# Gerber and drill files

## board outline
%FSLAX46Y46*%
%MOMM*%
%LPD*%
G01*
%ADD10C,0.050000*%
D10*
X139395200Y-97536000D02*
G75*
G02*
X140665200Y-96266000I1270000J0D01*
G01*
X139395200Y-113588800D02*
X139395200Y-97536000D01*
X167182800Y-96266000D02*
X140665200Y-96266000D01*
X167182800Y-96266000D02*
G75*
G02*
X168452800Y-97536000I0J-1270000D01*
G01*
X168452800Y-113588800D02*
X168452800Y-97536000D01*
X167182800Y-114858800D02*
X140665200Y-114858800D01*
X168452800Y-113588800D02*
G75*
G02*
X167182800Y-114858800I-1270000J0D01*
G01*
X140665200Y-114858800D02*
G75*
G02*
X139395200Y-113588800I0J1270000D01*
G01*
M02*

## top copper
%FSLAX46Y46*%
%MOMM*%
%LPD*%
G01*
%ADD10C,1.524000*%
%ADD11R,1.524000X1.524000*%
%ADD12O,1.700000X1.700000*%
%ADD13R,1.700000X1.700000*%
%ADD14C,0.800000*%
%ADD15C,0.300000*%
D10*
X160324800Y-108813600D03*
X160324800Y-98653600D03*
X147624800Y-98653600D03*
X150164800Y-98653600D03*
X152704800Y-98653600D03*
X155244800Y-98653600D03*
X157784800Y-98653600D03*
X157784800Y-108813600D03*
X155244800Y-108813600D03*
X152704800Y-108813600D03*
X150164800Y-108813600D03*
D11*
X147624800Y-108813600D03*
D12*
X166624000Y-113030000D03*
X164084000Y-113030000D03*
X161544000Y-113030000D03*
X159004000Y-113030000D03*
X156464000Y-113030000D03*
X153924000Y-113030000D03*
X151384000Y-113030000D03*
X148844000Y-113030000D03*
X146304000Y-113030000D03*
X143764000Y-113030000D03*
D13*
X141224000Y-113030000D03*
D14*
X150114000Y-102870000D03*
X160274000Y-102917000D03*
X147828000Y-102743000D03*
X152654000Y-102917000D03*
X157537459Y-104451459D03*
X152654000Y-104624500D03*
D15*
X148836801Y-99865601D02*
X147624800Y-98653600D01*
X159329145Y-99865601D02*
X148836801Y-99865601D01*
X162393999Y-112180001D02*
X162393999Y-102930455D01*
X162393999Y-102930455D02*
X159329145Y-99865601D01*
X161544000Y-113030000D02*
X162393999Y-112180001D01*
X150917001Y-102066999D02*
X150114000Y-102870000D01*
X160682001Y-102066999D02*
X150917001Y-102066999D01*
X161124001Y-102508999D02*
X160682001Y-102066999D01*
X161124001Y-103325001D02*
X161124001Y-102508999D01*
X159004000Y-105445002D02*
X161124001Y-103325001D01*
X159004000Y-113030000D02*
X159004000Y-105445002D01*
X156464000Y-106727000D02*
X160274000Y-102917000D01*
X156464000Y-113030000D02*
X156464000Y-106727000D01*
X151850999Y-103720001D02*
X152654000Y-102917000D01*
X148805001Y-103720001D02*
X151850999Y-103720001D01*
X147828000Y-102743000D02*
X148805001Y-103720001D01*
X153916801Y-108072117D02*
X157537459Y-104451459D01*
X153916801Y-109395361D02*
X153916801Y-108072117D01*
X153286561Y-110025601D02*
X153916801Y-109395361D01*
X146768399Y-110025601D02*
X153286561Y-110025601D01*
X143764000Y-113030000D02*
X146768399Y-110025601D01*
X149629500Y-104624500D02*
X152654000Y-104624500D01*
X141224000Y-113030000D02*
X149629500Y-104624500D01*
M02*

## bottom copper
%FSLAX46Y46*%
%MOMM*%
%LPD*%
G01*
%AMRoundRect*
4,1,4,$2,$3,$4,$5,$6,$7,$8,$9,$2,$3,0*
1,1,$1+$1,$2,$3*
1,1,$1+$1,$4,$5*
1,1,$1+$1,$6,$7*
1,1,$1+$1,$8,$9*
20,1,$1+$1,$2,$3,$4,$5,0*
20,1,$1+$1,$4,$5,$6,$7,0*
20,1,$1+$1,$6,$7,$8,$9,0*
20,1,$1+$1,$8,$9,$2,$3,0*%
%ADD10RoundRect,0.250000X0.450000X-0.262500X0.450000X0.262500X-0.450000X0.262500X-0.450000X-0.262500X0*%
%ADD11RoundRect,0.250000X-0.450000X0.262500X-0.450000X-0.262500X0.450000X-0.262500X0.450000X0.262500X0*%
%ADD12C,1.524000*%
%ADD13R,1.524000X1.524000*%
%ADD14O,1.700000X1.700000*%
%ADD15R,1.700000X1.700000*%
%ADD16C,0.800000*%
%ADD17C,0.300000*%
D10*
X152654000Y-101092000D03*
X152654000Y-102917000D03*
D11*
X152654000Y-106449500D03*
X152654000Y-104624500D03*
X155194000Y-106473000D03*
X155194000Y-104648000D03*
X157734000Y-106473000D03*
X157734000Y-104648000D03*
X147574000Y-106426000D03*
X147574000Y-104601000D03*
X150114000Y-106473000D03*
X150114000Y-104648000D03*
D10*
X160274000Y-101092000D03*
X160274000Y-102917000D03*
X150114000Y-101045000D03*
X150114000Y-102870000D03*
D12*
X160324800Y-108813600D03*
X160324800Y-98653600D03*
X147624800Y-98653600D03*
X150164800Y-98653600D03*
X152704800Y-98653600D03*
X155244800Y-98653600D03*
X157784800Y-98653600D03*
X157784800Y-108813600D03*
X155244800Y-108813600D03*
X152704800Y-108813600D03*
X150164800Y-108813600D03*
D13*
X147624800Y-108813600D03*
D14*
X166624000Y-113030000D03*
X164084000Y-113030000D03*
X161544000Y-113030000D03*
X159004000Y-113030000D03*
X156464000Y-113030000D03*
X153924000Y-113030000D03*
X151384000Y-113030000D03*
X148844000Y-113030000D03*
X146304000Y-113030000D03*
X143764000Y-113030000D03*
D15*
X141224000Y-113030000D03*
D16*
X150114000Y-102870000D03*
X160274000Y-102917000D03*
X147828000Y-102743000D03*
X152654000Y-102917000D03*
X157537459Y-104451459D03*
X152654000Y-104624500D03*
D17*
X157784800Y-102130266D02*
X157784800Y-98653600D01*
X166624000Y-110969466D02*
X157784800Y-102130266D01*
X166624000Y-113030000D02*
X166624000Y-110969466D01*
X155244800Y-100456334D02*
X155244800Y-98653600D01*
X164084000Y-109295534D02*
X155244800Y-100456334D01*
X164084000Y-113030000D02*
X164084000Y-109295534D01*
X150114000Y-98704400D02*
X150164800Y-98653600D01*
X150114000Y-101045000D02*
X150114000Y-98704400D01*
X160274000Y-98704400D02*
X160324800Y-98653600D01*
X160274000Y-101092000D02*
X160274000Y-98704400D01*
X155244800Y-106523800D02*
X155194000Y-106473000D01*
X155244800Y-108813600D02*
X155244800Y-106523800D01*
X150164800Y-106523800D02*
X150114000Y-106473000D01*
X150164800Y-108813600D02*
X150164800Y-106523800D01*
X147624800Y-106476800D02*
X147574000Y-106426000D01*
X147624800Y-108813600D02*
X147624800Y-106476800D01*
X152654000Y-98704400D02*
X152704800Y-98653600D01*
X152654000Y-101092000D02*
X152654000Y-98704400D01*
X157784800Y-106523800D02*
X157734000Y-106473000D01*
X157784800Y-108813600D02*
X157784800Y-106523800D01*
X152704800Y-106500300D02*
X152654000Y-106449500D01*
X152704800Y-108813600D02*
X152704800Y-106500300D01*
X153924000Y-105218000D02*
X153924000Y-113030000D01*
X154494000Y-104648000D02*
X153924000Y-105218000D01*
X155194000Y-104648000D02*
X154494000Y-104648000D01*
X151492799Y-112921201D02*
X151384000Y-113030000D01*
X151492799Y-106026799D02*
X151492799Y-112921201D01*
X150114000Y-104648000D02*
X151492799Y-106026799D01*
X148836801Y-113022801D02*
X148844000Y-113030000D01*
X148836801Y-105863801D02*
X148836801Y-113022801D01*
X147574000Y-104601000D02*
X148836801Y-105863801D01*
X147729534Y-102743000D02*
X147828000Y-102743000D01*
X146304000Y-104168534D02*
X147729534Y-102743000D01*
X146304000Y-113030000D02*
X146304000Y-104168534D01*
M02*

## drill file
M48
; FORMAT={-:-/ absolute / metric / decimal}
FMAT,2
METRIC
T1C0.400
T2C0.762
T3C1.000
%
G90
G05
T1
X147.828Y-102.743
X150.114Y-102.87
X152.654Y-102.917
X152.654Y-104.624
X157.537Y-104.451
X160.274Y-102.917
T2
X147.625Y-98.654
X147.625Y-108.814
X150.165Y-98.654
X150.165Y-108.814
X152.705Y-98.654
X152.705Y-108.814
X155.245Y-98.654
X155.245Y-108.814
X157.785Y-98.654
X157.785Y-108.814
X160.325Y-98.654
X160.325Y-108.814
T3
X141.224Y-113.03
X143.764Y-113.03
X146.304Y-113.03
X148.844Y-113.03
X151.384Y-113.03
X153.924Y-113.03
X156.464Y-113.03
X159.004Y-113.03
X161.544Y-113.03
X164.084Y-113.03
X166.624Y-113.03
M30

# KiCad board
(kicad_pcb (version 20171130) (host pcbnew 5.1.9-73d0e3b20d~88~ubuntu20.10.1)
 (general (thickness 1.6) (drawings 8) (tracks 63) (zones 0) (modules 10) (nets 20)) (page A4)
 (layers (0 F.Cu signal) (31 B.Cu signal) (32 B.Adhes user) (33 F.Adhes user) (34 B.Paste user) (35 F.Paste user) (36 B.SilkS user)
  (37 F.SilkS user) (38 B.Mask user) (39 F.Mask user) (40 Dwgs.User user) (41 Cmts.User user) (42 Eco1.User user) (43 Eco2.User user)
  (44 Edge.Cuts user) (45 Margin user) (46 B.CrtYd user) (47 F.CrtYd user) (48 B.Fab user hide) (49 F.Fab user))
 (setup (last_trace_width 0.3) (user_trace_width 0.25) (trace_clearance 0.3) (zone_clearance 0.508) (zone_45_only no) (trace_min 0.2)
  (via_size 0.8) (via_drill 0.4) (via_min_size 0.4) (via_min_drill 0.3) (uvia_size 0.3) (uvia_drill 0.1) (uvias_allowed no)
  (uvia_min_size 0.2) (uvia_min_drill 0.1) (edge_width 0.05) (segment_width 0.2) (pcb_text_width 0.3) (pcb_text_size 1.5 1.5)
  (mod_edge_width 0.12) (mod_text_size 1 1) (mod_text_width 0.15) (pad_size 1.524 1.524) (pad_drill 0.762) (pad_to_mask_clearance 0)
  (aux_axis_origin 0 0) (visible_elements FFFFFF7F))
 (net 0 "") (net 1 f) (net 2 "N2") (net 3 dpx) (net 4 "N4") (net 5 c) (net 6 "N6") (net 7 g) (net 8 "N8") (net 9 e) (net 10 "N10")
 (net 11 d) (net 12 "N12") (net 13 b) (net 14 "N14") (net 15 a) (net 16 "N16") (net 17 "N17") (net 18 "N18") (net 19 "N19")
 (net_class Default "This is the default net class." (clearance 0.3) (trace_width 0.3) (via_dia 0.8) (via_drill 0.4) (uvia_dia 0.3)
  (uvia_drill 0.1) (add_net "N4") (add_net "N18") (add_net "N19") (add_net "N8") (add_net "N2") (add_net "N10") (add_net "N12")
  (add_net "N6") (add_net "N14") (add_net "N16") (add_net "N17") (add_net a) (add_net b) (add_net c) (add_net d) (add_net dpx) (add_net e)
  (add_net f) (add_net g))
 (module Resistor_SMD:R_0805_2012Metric (layer B.Cu) (at 152.654 102.0045 90)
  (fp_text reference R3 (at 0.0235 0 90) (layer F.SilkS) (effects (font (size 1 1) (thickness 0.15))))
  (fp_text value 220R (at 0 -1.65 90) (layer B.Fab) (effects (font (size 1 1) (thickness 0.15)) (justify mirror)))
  (pad 2 smd roundrect (at 0.9125 0 90) (size 1.025 1.4) (layers B.Cu B.Paste B.Mask) (roundrect_rratio 0.243902) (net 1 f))
  (pad 1 smd roundrect (at -0.9125 0 90) (size 1.025 1.4) (layers B.Cu B.Paste B.Mask) (roundrect_rratio 0.243902) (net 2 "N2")))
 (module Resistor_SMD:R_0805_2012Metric (layer B.Cu) (at 152.654 105.537 270)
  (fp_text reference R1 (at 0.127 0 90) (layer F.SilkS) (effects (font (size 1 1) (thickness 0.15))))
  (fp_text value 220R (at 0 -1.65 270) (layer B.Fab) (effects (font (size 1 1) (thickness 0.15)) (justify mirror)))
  (pad 2 smd roundrect (at 0.9125 0 270) (size 1.025 1.4) (layers B.Cu B.Paste B.Mask) (roundrect_rratio 0.243902) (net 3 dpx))
  (pad 1 smd roundrect (at -0.9125 0 270) (size 1.025 1.4) (layers B.Cu B.Paste B.Mask) (roundrect_rratio 0.243902) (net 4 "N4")))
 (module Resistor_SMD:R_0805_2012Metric (layer B.Cu) (at 155.194 105.5605 270)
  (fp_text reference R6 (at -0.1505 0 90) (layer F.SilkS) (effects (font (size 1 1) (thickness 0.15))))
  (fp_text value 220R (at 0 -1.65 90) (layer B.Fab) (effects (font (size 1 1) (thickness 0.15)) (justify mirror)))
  (pad 2 smd roundrect (at 0.9125 0 270) (size 1.025 1.4) (layers B.Cu B.Paste B.Mask) (roundrect_rratio 0.243902) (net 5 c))
  (pad 1 smd roundrect (at -0.9125 0 270) (size 1.025 1.4) (layers B.Cu B.Paste B.Mask) (roundrect_rratio 0.243902) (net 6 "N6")))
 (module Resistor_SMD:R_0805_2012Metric (layer B.Cu) (at 157.734 105.5605 270)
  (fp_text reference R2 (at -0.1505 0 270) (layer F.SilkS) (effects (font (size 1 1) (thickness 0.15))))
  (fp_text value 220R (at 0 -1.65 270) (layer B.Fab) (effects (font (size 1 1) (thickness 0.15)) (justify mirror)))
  (pad 2 smd roundrect (at 0.9125 0 270) (size 1.025 1.4) (layers B.Cu B.Paste B.Mask) (roundrect_rratio 0.243902) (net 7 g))
  (pad 1 smd roundrect (at -0.9125 0 270) (size 1.025 1.4) (layers B.Cu B.Paste B.Mask) (roundrect_rratio 0.243902) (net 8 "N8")))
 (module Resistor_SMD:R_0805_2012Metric (layer B.Cu) (at 147.574 105.5135 270)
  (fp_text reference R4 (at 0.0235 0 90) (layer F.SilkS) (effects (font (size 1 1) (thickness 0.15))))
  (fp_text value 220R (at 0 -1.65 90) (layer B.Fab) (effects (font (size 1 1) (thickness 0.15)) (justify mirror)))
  (pad 2 smd roundrect (at 0.9125 0 270) (size 1.025 1.4) (layers B.Cu B.Paste B.Mask) (roundrect_rratio 0.243902) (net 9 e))
  (pad 1 smd roundrect (at -0.9125 0 270) (size 1.025 1.4) (layers B.Cu B.Paste B.Mask) (roundrect_rratio 0.243902) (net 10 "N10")))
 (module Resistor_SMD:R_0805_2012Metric (layer B.Cu) (at 150.114 105.5605 270)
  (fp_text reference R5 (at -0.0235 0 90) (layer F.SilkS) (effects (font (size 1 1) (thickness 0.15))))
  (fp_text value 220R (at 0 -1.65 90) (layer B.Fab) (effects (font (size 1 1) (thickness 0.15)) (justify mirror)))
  (pad 2 smd roundrect (at 0.9125 0 270) (size 1.025 1.4) (layers B.Cu B.Paste B.Mask) (roundrect_rratio 0.243902) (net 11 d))
  (pad 1 smd roundrect (at -0.9125 0 270) (size 1.025 1.4) (layers B.Cu B.Paste B.Mask) (roundrect_rratio 0.243902) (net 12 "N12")))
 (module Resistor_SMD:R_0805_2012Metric (layer B.Cu) (at 160.274 102.0045 90)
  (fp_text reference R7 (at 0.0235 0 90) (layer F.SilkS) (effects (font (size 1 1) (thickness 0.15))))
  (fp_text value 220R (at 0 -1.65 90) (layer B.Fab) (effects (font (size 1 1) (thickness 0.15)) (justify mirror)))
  (pad 2 smd roundrect (at 0.9125 0 90) (size 1.025 1.4) (layers B.Cu B.Paste B.Mask) (roundrect_rratio 0.243902) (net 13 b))
  (pad 1 smd roundrect (at -0.9125 0 90) (size 1.025 1.4) (layers B.Cu B.Paste B.Mask) (roundrect_rratio 0.243902) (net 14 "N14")))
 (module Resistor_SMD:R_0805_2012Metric (layer B.Cu) (at 150.114 101.9575 90)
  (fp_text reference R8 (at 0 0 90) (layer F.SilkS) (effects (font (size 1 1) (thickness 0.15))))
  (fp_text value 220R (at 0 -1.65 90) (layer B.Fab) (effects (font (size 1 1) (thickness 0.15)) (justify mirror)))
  (pad 2 smd roundrect (at 0.9125 0 90) (size 1.025 1.4) (layers B.Cu B.Paste B.Mask) (roundrect_rratio 0.243902) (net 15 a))
  (pad 1 smd roundrect (at -0.9125 0 90) (size 1.025 1.4) (layers B.Cu B.Paste B.Mask) (roundrect_rratio 0.243902) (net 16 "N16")))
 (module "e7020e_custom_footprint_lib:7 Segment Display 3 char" (layer F.Cu) (at 147.6248 98.6536)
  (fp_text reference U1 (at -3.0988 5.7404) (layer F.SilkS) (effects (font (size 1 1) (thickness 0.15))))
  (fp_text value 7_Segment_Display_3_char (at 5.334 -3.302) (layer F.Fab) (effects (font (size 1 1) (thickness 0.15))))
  (pad 6 thru_hole circle (at 12.7 10.16) (size 1.524 1.524) (drill 0.762) (layers *.Cu *.Mask))
  (pad 7 thru_hole circle (at 12.7 0) (size 1.524 1.524) (drill 0.762) (layers *.Cu *.Mask) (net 13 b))
  (pad 12 thru_hole circle (at 0 0) (size 1.524 1.524) (drill 0.762) (layers *.Cu *.Mask) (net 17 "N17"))
  (pad 11 thru_hole circle (at 2.54 0) (size 1.524 1.524) (drill 0.762) (layers *.Cu *.Mask) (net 15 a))
  (pad 10 thru_hole circle (at 5.08 0) (size 1.524 1.524) (drill 0.762) (layers *.Cu *.Mask) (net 1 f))
  (pad 9 thru_hole circle (at 7.62 0) (size 1.524 1.524) (drill 0.762) (layers *.Cu *.Mask) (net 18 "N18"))
  (pad 8 thru_hole circle (at 10.16 0) (size 1.524 1.524) (drill 0.762) (layers *.Cu *.Mask) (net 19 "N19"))
  (pad 5 thru_hole circle (at 10.16 10.16) (size 1.524 1.524) (drill 0.762) (layers *.Cu *.Mask) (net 7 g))
  (pad 4 thru_hole circle (at 7.62 10.16) (size 1.524 1.524) (drill 0.762) (layers *.Cu *.Mask) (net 5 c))
  (pad 3 thru_hole circle (at 5.08 10.16) (size 1.524 1.524) (drill 0.762) (layers *.Cu *.Mask) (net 3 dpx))
  (pad 2 thru_hole circle (at 2.54 10.16) (size 1.524 1.524) (drill 0.762) (layers *.Cu *.Mask) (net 11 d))
  (pad 1 thru_hole rect (at 0 10.16) (size 1.524 1.524) (drill 0.762) (layers *.Cu *.Mask) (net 9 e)))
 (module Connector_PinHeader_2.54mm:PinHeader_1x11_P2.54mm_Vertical (layer B.Cu) (at 141.224 113.03 270)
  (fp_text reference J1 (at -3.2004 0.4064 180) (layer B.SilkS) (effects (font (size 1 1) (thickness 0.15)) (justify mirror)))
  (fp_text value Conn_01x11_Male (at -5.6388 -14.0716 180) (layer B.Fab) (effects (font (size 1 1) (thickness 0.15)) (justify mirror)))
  (pad 11 thru_hole oval (at 0 -25.4 270) (size 1.7 1.7) (drill 1) (layers *.Cu *.Mask) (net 19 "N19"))
  (pad 10 thru_hole oval (at 0 -22.86 270) (size 1.7 1.7) (drill 1) (layers *.Cu *.Mask) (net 18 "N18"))
  (pad 9 thru_hole oval (at 0 -20.32 270) (size 1.7 1.7) (drill 1) (layers *.Cu *.Mask) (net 17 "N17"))
  (pad 8 thru_hole oval (at 0 -17.78 270) (size 1.7 1.7) (drill 1) (layers *.Cu *.Mask) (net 16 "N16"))
  (pad 7 thru_hole oval (at 0 -15.24 270) (size 1.7 1.7) (drill 1) (layers *.Cu *.Mask) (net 14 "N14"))
  (pad 6 thru_hole oval (at 0 -12.7 270) (size 1.7 1.7) (drill 1) (layers *.Cu *.Mask) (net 6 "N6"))
  (pad 5 thru_hole oval (at 0 -10.16 270) (size 1.7 1.7) (drill 1) (layers *.Cu *.Mask) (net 12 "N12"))
  (pad 4 thru_hole oval (at 0 -7.62 270) (size 1.7 1.7) (drill 1) (layers *.Cu *.Mask) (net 10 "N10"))
  (pad 3 thru_hole oval (at 0 -5.08 270) (size 1.7 1.7) (drill 1) (layers *.Cu *.Mask) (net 2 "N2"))
  (pad 2 thru_hole oval (at 0 -2.54 270) (size 1.7 1.7) (drill 1) (layers *.Cu *.Mask) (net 8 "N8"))
  (pad 1 thru_hole rect (at 0 0 270) (size 1.7 1.7) (drill 1) (layers *.Cu *.Mask) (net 4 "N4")))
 (gr_arc (start 140.6652 97.536) (end 140.6652 96.266) (angle -90) (layer Edge.Cuts) (width 0.05))
 (gr_line (start 139.3952 113.5888) (end 139.3952 97.536) (layer Edge.Cuts) (width 0.05))
 (gr_line (start 167.1828 96.266) (end 140.6652 96.266) (layer Edge.Cuts) (width 0.05))
 (gr_arc (start 167.1828 97.536) (end 168.4528 97.536) (angle -90) (layer Edge.Cuts) (width 0.05))
 (gr_line (start 168.4528 113.5888) (end 168.4528 97.536) (layer Edge.Cuts) (width 0.05))
 (gr_line (start 167.1828 114.8588) (end 140.6652 114.8588) (layer Edge.Cuts) (width 0.05))
 (gr_arc (start 167.1828 113.5888) (end 167.1828 114.8588) (angle -90) (layer Edge.Cuts) (width 0.05))
 (gr_arc (start 140.6652 113.5888) (end 139.3952 113.5888) (angle -90) (layer Edge.Cuts) (width 0.05))
 (segment (start 157.7848 102.130266) (end 157.7848 98.6536) (width 0.3) (layer B.Cu) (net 19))
 (segment (start 166.624 110.969466) (end 157.7848 102.130266) (width 0.3) (layer B.Cu) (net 19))
 (segment (start 166.624 113.03) (end 166.624 110.969466) (width 0.3) (layer B.Cu) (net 19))
 (segment (start 155.2448 100.456334) (end 155.2448 98.6536) (width 0.3) (layer B.Cu) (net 18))
 (segment (start 164.084 109.295534) (end 155.2448 100.456334) (width 0.3) (layer B.Cu) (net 18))
 (segment (start 164.084 113.03) (end 164.084 109.295534) (width 0.3) (layer B.Cu) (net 18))
 (segment (start 148.836801 99.865601) (end 147.6248 98.6536) (width 0.3) (layer F.Cu) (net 17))
 (segment (start 159.329145 99.865601) (end 148.836801 99.865601) (width 0.3) (layer F.Cu) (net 17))
 (segment (start 162.393999 112.180001) (end 162.393999 102.930455) (width 0.3) (layer F.Cu) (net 17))
 (segment (start 162.393999 102.930455) (end 159.329145 99.865601) (width 0.3) (layer F.Cu) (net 17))
 (segment (start 161.544 113.03) (end 162.393999 112.180001) (width 0.3) (layer F.Cu) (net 17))
 (segment (start 150.114 98.7044) (end 150.1648 98.6536) (width 0.3) (layer B.Cu) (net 15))
 (segment (start 150.114 101.045) (end 150.114 98.7044) (width 0.3) (layer B.Cu) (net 15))
 (segment (start 160.274 98.7044) (end 160.3248 98.6536) (width 0.3) (layer B.Cu) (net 13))
 (segment (start 160.274 101.092) (end 160.274 98.7044) (width 0.3) (layer B.Cu) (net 13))
 (segment (start 155.2448 106.5238) (end 155.194 106.473) (width 0.3) (layer B.Cu) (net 5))
 (segment (start 155.2448 108.8136) (end 155.2448 106.5238) (width 0.3) (layer B.Cu) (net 5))
 (segment (start 150.1648 106.5238) (end 150.114 106.473) (width 0.3) (layer B.Cu) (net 11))
 (segment (start 150.1648 108.8136) (end 150.1648 106.5238) (width 0.3) (layer B.Cu) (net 11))
 (segment (start 147.6248 106.4768) (end 147.574 106.426) (width 0.3) (layer B.Cu) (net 9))
 (segment (start 147.6248 108.8136) (end 147.6248 106.4768) (width 0.3) (layer B.Cu) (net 9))
 (segment (start 152.654 98.7044) (end 152.7048 98.6536) (width 0.3) (layer B.Cu) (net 1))
 (segment (start 152.654 101.092) (end 152.654 98.7044) (width 0.3) (layer B.Cu) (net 1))
 (segment (start 157.7848 106.5238) (end 157.734 106.473) (width 0.3) (layer B.Cu) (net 7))
 (segment (start 157.7848 108.8136) (end 157.7848 106.5238) (width 0.3) (layer B.Cu) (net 7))
 (segment (start 152.7048 106.5003) (end 152.654 106.4495) (width 0.3) (layer B.Cu) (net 3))
 (segment (start 152.7048 108.8136) (end 152.7048 106.5003) (width 0.3) (layer B.Cu) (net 3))
 (segment (start 150.917001 102.066999) (end 150.114 102.87) (width 0.3) (layer F.Cu) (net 16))
 (segment (start 160.682001 102.066999) (end 150.917001 102.066999) (width 0.3) (layer F.Cu) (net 16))
 (segment (start 161.124001 102.508999) (end 160.682001 102.066999) (width 0.3) (layer F.Cu) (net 16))
 (segment (start 161.124001 103.325001) (end 161.124001 102.508999) (width 0.3) (layer F.Cu) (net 16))
 (segment (start 159.004 105.445002) (end 161.124001 103.325001) (width 0.3) (layer F.Cu) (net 16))
 (via (at 150.114 102.87) (size 0.8) (drill 0.4) (layers F.Cu B.Cu) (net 16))
 (segment (start 159.004 113.03) (end 159.004 105.445002) (width 0.3) (layer F.Cu) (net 16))
 (via (at 160.274 102.917) (size 0.8) (drill 0.4) (layers F.Cu B.Cu) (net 14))
 (segment (start 156.464 106.727) (end 160.274 102.917) (width 0.3) (layer F.Cu) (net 14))
 (segment (start 156.464 113.03) (end 156.464 106.727) (width 0.3) (layer F.Cu) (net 14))
 (segment (start 153.924 105.218) (end 153.924 113.03) (width 0.3) (layer B.Cu) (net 6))
 (segment (start 154.494 104.648) (end 153.924 105.218) (width 0.3) (layer B.Cu) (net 6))
 (segment (start 155.194 104.648) (end 154.494 104.648) (width 0.3) (layer B.Cu) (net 6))
 (segment (start 151.492799 112.921201) (end 151.384 113.03) (width 0.3) (layer B.Cu) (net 12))
 (segment (start 151.492799 106.026799) (end 151.492799 112.921201) (width 0.3) (layer B.Cu) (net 12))
 (segment (start 150.114 104.648) (end 151.492799 106.026799) (width 0.3) (layer B.Cu) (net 12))
 (segment (start 148.836801 113.022801) (end 148.844 113.03) (width 0.3) (layer B.Cu) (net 10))
 (segment (start 148.836801 105.863801) (end 148.836801 113.022801) (width 0.3) (layer B.Cu) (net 10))
 (segment (start 147.574 104.601) (end 148.836801 105.863801) (width 0.3) (layer B.Cu) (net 10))
 (via (at 147.828 102.743) (size 0.8) (drill 0.4) (layers F.Cu B.Cu) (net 2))
 (segment (start 147.729534 102.743) (end 147.828 102.743) (width 0.3) (layer B.Cu) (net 2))
 (segment (start 146.304 104.168534) (end 147.729534 102.743) (width 0.3) (layer B.Cu) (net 2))
 (segment (start 146.304 113.03) (end 146.304 104.168534) (width 0.3) (layer B.Cu) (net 2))
 (via (at 152.654 102.917) (size 0.8) (drill 0.4) (layers F.Cu B.Cu) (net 2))
 (segment (start 151.850999 103.720001) (end 152.654 102.917) (width 0.3) (layer F.Cu) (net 2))
 (segment (start 148.805001 103.720001) (end 151.850999 103.720001) (width 0.3) (layer F.Cu) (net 2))
 (segment (start 147.828 102.743) (end 148.805001 103.720001) (width 0.3) (layer F.Cu) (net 2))
 (via (at 157.537459 104.451459) (size 0.8) (drill 0.4) (layers F.Cu B.Cu) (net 8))
 (segment (start 153.916801 108.072117) (end 157.537459 104.451459) (width 0.3) (layer F.Cu) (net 8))
 (segment (start 153.916801 109.395361) (end 153.916801 108.072117) (width 0.3) (layer F.Cu) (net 8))
 (segment (start 153.286561 110.025601) (end 153.916801 109.395361) (width 0.3) (layer F.Cu) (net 8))
 (segment (start 146.768399 110.025601) (end 153.286561 110.025601) (width 0.3) (layer F.Cu) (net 8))
 (segment (start 143.764 113.03) (end 146.768399 110.025601) (width 0.3) (layer F.Cu) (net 8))
 (via (at 152.654 104.6245) (size 0.8) (drill 0.4) (layers F.Cu B.Cu) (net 4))
 (segment (start 149.6295 104.6245) (end 152.654 104.6245) (width 0.3) (layer F.Cu) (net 4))
 (segment (start 141.224 113.03) (end 149.6295 104.6245) (width 0.3) (layer F.Cu) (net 4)))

